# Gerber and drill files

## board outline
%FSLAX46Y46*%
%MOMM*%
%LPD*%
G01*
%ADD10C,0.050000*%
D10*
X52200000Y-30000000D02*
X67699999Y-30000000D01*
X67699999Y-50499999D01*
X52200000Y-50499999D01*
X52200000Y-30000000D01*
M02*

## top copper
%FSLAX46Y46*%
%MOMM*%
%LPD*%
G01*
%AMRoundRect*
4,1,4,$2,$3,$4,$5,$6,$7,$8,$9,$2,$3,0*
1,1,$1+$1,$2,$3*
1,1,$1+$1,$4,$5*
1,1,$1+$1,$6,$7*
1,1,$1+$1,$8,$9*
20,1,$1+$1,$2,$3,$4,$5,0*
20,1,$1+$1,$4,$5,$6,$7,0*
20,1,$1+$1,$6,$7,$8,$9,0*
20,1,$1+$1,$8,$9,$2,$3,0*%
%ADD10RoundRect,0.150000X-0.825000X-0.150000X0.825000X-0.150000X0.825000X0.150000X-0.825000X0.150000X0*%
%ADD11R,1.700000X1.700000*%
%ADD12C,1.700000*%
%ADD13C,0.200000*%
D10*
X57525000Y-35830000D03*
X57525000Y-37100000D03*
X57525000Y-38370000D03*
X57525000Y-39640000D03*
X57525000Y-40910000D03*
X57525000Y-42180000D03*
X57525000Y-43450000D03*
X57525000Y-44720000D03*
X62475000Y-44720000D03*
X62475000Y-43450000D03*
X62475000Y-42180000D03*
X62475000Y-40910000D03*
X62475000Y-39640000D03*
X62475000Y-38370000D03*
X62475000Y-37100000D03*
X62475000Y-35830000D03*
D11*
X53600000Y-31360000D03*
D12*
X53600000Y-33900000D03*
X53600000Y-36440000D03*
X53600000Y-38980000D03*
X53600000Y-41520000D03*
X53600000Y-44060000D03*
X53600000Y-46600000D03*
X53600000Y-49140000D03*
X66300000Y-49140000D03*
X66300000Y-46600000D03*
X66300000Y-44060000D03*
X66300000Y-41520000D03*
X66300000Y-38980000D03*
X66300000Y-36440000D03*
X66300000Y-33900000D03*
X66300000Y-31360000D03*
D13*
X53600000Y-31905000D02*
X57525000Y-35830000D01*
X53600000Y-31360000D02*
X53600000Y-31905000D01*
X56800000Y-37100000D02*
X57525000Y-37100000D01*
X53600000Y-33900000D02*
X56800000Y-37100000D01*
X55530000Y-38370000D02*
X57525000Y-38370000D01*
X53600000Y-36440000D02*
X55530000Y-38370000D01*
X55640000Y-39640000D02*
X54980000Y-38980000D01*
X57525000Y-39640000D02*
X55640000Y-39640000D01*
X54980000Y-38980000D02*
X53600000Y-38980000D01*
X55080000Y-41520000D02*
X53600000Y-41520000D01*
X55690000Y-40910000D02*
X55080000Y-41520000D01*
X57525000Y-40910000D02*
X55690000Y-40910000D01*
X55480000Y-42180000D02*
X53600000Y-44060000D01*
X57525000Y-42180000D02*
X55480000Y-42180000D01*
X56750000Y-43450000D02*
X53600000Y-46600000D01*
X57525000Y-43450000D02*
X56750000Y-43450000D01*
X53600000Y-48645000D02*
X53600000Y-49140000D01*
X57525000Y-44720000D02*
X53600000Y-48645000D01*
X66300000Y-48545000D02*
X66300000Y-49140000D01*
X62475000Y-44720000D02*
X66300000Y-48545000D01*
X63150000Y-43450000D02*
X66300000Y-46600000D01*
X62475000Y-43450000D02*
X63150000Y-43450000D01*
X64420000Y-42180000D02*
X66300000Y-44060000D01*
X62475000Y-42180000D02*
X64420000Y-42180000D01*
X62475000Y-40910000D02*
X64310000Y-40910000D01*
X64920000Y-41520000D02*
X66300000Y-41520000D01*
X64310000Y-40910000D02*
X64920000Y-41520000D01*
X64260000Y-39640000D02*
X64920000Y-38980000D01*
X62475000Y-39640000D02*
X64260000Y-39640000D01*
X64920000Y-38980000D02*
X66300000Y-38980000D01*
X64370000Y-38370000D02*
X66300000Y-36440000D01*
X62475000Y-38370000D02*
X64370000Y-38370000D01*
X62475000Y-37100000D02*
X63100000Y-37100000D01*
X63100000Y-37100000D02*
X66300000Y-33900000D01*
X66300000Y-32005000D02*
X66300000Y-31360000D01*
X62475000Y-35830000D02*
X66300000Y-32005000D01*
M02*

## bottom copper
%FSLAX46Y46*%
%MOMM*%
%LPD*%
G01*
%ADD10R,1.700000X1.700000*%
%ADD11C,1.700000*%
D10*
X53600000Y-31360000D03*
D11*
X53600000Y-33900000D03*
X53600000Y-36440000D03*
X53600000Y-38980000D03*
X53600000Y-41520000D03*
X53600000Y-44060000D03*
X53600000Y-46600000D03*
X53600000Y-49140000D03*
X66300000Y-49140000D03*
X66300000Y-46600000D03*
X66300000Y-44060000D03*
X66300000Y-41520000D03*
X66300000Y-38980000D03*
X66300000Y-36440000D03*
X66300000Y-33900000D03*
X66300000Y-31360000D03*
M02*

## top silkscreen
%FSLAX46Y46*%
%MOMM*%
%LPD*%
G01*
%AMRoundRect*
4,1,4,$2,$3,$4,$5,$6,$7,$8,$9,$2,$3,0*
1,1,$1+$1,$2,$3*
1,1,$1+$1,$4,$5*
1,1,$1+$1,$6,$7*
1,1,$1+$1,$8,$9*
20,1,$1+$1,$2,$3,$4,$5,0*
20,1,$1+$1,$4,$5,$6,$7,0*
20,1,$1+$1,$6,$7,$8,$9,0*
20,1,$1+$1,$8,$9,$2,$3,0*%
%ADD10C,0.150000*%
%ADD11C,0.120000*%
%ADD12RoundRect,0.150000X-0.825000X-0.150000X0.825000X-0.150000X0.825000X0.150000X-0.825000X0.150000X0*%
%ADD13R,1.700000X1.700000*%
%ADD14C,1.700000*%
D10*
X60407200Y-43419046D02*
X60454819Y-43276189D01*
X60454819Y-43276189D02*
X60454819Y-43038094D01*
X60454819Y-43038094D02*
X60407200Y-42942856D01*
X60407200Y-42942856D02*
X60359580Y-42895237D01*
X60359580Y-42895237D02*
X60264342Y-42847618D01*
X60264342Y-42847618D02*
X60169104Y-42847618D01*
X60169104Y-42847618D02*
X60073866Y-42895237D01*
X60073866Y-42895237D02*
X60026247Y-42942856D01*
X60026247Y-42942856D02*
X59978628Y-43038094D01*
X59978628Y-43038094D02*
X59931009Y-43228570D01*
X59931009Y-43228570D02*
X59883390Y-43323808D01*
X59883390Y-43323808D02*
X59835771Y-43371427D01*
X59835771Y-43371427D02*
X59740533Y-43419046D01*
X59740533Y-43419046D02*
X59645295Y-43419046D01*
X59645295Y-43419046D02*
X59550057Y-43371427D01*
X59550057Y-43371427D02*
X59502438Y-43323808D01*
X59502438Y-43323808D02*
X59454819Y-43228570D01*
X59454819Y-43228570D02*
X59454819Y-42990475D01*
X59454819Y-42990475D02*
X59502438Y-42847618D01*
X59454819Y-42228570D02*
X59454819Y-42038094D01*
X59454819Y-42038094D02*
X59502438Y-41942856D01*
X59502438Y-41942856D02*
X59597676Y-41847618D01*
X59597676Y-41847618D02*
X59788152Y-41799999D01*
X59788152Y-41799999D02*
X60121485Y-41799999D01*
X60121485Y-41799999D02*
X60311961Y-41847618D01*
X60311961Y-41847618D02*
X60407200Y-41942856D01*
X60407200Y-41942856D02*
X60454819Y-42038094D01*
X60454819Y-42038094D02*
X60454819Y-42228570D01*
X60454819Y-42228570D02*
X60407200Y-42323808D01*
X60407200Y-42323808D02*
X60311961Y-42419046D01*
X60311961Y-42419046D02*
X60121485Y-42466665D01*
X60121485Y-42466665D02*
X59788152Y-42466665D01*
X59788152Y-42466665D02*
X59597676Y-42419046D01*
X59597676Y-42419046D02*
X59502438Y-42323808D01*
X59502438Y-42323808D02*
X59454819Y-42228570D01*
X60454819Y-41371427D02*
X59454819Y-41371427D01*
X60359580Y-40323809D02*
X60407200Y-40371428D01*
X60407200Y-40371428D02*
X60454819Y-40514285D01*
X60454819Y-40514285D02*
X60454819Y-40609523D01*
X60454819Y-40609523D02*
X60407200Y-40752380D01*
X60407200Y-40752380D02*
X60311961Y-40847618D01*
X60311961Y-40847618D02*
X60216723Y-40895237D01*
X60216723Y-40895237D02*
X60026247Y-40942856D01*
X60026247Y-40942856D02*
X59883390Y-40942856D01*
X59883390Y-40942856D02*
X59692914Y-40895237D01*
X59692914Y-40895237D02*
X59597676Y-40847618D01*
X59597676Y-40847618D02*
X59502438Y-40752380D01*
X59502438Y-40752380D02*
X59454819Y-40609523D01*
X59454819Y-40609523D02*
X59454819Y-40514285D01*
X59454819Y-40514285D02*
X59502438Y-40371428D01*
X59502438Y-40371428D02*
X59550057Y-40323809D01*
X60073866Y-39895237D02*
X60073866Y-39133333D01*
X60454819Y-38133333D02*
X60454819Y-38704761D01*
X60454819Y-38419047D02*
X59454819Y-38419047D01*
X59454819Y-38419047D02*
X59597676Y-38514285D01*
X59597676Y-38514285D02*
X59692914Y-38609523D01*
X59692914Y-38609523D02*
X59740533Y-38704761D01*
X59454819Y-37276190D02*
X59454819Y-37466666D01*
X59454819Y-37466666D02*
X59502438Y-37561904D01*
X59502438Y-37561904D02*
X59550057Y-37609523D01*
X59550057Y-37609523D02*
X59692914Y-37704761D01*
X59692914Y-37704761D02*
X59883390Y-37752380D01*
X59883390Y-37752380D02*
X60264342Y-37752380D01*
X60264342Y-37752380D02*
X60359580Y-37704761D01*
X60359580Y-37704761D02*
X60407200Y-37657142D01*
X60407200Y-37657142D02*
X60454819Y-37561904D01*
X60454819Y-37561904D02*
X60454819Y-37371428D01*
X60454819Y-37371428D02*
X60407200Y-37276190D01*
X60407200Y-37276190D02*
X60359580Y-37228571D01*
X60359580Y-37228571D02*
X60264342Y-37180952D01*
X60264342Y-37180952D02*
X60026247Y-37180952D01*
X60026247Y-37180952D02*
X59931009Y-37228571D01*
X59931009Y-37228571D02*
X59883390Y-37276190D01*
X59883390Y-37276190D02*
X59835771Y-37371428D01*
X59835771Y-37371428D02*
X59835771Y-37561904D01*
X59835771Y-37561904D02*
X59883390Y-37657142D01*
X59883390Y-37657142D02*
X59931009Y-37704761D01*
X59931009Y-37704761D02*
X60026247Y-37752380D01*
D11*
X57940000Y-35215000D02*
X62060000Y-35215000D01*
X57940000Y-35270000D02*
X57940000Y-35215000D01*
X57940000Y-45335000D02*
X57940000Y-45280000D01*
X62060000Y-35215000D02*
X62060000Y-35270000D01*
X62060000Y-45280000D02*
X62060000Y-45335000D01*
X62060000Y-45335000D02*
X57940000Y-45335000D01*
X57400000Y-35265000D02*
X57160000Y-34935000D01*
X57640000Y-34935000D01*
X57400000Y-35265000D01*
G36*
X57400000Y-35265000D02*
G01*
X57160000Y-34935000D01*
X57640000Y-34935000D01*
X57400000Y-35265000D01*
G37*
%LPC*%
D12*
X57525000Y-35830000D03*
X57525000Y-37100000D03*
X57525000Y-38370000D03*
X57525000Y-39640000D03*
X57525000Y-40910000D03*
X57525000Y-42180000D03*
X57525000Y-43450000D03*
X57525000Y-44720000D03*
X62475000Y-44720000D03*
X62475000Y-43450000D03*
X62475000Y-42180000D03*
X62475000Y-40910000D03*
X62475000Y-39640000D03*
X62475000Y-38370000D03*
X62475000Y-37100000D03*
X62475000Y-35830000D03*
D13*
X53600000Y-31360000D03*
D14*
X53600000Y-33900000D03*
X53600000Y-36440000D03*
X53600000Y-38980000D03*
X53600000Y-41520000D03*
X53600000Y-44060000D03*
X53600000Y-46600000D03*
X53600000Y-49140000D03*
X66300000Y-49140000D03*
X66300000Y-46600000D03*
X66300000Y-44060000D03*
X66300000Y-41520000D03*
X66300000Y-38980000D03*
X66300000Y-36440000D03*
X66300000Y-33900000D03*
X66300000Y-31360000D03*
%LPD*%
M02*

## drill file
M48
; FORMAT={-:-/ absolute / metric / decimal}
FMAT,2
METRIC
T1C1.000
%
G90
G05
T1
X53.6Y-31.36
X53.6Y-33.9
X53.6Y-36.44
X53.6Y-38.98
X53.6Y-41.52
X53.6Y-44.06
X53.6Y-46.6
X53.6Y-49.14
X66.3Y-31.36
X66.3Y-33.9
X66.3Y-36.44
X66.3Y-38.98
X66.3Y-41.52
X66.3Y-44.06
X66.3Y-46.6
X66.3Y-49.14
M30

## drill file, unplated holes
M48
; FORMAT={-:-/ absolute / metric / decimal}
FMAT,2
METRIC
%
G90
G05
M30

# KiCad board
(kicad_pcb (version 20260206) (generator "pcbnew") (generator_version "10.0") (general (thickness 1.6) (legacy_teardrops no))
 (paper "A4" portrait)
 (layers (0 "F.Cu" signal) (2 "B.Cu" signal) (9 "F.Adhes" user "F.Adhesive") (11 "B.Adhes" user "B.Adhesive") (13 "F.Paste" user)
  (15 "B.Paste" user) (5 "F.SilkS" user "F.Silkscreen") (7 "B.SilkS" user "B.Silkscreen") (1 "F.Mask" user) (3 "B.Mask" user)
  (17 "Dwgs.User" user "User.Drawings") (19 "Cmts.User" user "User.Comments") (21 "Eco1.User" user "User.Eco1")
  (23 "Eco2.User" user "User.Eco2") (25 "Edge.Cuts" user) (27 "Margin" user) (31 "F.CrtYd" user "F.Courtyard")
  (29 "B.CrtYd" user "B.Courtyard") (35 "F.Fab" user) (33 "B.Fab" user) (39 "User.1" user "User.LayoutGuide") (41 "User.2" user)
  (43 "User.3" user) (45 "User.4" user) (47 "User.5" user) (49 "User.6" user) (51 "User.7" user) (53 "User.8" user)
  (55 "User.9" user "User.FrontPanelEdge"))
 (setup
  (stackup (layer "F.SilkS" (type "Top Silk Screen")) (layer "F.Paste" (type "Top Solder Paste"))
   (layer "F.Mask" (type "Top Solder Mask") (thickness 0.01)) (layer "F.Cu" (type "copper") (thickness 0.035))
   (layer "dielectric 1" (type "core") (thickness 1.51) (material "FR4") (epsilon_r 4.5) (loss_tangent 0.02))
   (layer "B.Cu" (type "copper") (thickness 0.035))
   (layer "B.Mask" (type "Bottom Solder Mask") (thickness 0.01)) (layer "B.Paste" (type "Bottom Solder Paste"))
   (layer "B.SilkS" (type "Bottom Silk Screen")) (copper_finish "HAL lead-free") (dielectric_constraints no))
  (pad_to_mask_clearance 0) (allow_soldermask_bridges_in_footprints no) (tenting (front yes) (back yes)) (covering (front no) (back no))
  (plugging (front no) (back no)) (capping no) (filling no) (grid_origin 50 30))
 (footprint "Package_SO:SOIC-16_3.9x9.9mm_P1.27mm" (layer "F.Cu") (at 60 40.275)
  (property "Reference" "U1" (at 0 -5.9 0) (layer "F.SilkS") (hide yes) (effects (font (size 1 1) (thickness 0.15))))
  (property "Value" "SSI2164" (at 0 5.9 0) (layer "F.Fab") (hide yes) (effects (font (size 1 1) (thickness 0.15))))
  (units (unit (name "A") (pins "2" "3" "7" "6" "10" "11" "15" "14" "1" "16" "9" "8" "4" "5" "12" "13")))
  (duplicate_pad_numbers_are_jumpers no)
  (fp_line (start -2.06 -5.06) (end 2.06 -5.06) (stroke (width 0.12) (type solid)) (layer "F.SilkS"))
  (fp_line (start -2.06 -5.005) (end -2.06 -5.06) (stroke (width 0.12) (type solid)) (layer "F.SilkS"))
  (fp_line (start -2.06 5.06) (end -2.06 5.005) (stroke (width 0.12) (type solid)) (layer "F.SilkS"))
  (fp_line (start 2.06 -5.06) (end 2.06 -5.005) (stroke (width 0.12) (type solid)) (layer "F.SilkS"))
  (fp_line (start 2.06 5.005) (end 2.06 5.06) (stroke (width 0.12) (type solid)) (layer "F.SilkS"))
  (fp_line (start 2.06 5.06) (end -2.06 5.06) (stroke (width 0.12) (type solid)) (layer "F.SilkS"))
  (fp_poly (pts (xy -2.6 -5.01) (xy -2.84 -5.34) (xy -2.36 -5.34)) (stroke (width 0.12) (type solid)) (fill yes) (layer "F.SilkS"))
  (pad "1" smd roundrect (at -2.475 -4.445) (size 1.95 0.6) (layers "F.Cu" "F.Mask" "F.Paste") (roundrect_rratio 0.25)
   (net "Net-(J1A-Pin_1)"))
  (pad "2" smd roundrect (at -2.475 -3.175) (size 1.95 0.6) (layers "F.Cu" "F.Mask" "F.Paste") (roundrect_rratio 0.25)
   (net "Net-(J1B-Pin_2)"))
  (pad "3" smd roundrect (at -2.475 -1.905) (size 1.95 0.6) (layers "F.Cu" "F.Mask" "F.Paste") (roundrect_rratio 0.25)
   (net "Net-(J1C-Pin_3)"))
  (pad "4" smd roundrect (at -2.475 -0.635) (size 1.95 0.6) (layers "F.Cu" "F.Mask" "F.Paste") (roundrect_rratio 0.25)
   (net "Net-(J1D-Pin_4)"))
  (pad "5" smd roundrect (at -2.475 0.635) (size 1.95 0.6) (layers "F.Cu" "F.Mask" "F.Paste") (roundrect_rratio 0.25)
   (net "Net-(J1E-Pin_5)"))
  (pad "6" smd roundrect (at -2.475 1.905) (size 1.95 0.6) (layers "F.Cu" "F.Mask" "F.Paste") (roundrect_rratio 0.25)
   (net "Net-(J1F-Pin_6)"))
  (pad "7" smd roundrect (at -2.475 3.175) (size 1.95 0.6) (layers "F.Cu" "F.Mask" "F.Paste") (roundrect_rratio 0.25)
   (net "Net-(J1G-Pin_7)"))
  (pad "8" smd roundrect (at -2.475 4.445) (size 1.95 0.6) (layers "F.Cu" "F.Mask" "F.Paste") (roundrect_rratio 0.25)
   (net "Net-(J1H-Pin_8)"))
  (pad "9" smd roundrect (at 2.475 4.445) (size 1.95 0.6) (layers "F.Cu" "F.Mask" "F.Paste") (roundrect_rratio 0.25) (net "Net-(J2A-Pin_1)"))
  (pad "10" smd roundrect (at 2.475 3.175) (size 1.95 0.6) (layers "F.Cu" "F.Mask" "F.Paste") (roundrect_rratio 0.25)
   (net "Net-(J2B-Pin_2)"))
  (pad "11" smd roundrect (at 2.475 1.905) (size 1.95 0.6) (layers "F.Cu" "F.Mask" "F.Paste") (roundrect_rratio 0.25)
   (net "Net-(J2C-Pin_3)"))
  (pad "12" smd roundrect (at 2.475 0.635) (size 1.95 0.6) (layers "F.Cu" "F.Mask" "F.Paste") (roundrect_rratio 0.25)
   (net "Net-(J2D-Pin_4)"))
  (pad "13" smd roundrect (at 2.475 -0.635) (size 1.95 0.6) (layers "F.Cu" "F.Mask" "F.Paste") (roundrect_rratio 0.25)
   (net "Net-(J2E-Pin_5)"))
  (pad "14" smd roundrect (at 2.475 -1.905) (size 1.95 0.6) (layers "F.Cu" "F.Mask" "F.Paste") (roundrect_rratio 0.25)
   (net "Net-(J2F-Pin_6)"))
  (pad "15" smd roundrect (at 2.475 -3.175) (size 1.95 0.6) (layers "F.Cu" "F.Mask" "F.Paste") (roundrect_rratio 0.25)
   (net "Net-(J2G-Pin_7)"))
  (pad "16" smd roundrect (at 2.475 -4.445) (size 1.95 0.6) (layers "F.Cu" "F.Mask" "F.Paste") (roundrect_rratio 0.25)
   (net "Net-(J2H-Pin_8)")))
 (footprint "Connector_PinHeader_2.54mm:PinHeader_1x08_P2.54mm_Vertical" (layer "B.Cu") (at 53.6 31.36 180)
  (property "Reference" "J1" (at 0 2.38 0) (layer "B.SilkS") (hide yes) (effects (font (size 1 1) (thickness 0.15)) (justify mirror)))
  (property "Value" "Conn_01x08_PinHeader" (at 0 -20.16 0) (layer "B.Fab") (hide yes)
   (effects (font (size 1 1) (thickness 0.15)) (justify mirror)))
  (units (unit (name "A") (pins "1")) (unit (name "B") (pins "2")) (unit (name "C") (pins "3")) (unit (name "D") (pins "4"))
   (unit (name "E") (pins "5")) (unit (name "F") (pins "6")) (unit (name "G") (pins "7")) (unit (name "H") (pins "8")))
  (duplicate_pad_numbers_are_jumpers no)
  (pad "1" thru_hole rect (at 0 0 180) (size 1.7 1.7) (drill 1) (layers "*.Cu" "*.Mask") (remove_unused_layers no) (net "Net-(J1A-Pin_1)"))
  (pad "2" thru_hole circle (at 0 -2.54 180) (size 1.7 1.7) (drill 1) (layers "*.Cu" "*.Mask") (remove_unused_layers no)
   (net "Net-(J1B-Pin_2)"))
  (pad "3" thru_hole circle (at 0 -5.08 180) (size 1.7 1.7) (drill 1) (layers "*.Cu" "*.Mask") (remove_unused_layers no)
   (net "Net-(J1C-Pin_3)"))
  (pad "4" thru_hole circle (at 0 -7.62 180) (size 1.7 1.7) (drill 1) (layers "*.Cu" "*.Mask") (remove_unused_layers no)
   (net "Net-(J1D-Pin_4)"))
  (pad "5" thru_hole circle (at 0 -10.16 180) (size 1.7 1.7) (drill 1) (layers "*.Cu" "*.Mask") (remove_unused_layers no)
   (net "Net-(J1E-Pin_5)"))
  (pad "6" thru_hole circle (at 0 -12.7 180) (size 1.7 1.7) (drill 1) (layers "*.Cu" "*.Mask") (remove_unused_layers no)
   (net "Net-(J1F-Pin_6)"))
  (pad "7" thru_hole circle (at 0 -15.24 180) (size 1.7 1.7) (drill 1) (layers "*.Cu" "*.Mask") (remove_unused_layers no)
   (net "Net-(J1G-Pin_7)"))
  (pad "8" thru_hole circle (at 0 -17.78 180) (size 1.7 1.7) (drill 1) (layers "*.Cu" "*.Mask") (remove_unused_layers no)
   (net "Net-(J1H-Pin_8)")))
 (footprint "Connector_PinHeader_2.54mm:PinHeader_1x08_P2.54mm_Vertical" (layer "B.Cu") (at 66.3 49.14)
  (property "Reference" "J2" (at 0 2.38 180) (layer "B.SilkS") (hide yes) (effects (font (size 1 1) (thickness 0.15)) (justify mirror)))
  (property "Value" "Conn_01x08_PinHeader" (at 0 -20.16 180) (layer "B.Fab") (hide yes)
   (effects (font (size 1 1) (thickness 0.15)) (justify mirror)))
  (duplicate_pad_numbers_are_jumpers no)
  (pad "1" thru_hole circle (at 0 0) (size 1.7 1.7) (drill 1) (layers "*.Cu" "*.Mask") (remove_unused_layers no) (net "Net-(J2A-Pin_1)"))
  (pad "2" thru_hole circle (at 0 -2.54) (size 1.7 1.7) (drill 1) (layers "*.Cu" "*.Mask") (remove_unused_layers no) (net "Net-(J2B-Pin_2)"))
  (pad "3" thru_hole circle (at 0 -5.08) (size 1.7 1.7) (drill 1) (layers "*.Cu" "*.Mask") (remove_unused_layers no) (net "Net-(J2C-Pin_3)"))
  (pad "4" thru_hole circle (at 0 -7.62) (size 1.7 1.7) (drill 1) (layers "*.Cu" "*.Mask") (remove_unused_layers no) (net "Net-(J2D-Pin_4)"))
  (pad "5" thru_hole circle (at 0 -10.16) (size 1.7 1.7) (drill 1) (layers "*.Cu" "*.Mask") (remove_unused_layers no)
   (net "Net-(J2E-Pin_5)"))
  (pad "6" thru_hole circle (at 0 -12.7) (size 1.7 1.7) (drill 1) (layers "*.Cu" "*.Mask") (remove_unused_layers no) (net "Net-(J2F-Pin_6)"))
  (pad "7" thru_hole circle (at 0 -15.24) (size 1.7 1.7) (drill 1) (layers "*.Cu" "*.Mask") (remove_unused_layers no)
   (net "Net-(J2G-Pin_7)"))
  (pad "8" thru_hole circle (at 0 -17.78) (size 1.7 1.7) (drill 1) (layers "*.Cu" "*.Mask") (remove_unused_layers no)
   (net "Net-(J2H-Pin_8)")))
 (gr_rect (start 52.2 30) (end 67.699999 50.499999) (stroke (width 0.05) (type default)) (fill no) (layer "Edge.Cuts"))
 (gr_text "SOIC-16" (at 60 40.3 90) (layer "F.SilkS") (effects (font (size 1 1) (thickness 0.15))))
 (segment (start 53.6 31.905) (end 57.525 35.83) (width 0.2) (layer "F.Cu") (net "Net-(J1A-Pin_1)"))
 (segment (start 53.6 31.36) (end 53.6 31.905) (width 0.2) (layer "F.Cu") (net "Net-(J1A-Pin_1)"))
 (segment (start 56.8 37.1) (end 57.525 37.1) (width 0.2) (layer "F.Cu") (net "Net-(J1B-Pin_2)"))
 (segment (start 53.6 33.9) (end 56.8 37.1) (width 0.2) (layer "F.Cu") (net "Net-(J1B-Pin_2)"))
 (segment (start 55.53 38.37) (end 57.525 38.37) (width 0.2) (layer "F.Cu") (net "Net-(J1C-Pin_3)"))
 (segment (start 53.6 36.44) (end 55.53 38.37) (width 0.2) (layer "F.Cu") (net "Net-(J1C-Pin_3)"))
 (segment (start 55.64 39.64) (end 54.98 38.98) (width 0.2) (layer "F.Cu") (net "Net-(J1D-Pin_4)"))
 (segment (start 57.525 39.64) (end 55.64 39.64) (width 0.2) (layer "F.Cu") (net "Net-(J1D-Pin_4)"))
 (segment (start 54.98 38.98) (end 53.6 38.98) (width 0.2) (layer "F.Cu") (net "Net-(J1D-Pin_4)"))
 (segment (start 55.08 41.52) (end 53.6 41.52) (width 0.2) (layer "F.Cu") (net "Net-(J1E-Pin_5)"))
 (segment (start 55.69 40.91) (end 55.08 41.52) (width 0.2) (layer "F.Cu") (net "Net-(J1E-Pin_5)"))
 (segment (start 57.525 40.91) (end 55.69 40.91) (width 0.2) (layer "F.Cu") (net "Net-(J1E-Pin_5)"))
 (segment (start 55.48 42.18) (end 53.6 44.06) (width 0.2) (layer "F.Cu") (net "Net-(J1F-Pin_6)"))
 (segment (start 57.525 42.18) (end 55.48 42.18) (width 0.2) (layer "F.Cu") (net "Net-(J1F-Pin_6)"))
 (segment (start 56.75 43.45) (end 53.6 46.6) (width 0.2) (layer "F.Cu") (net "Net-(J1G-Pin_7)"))
 (segment (start 57.525 43.45) (end 56.75 43.45) (width 0.2) (layer "F.Cu") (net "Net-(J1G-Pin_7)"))
 (segment (start 53.6 48.645) (end 53.6 49.14) (width 0.2) (layer "F.Cu") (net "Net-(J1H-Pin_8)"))
 (segment (start 57.525 44.72) (end 53.6 48.645) (width 0.2) (layer "F.Cu") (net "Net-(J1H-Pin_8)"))
 (segment (start 66.3 48.545) (end 66.3 49.14) (width 0.2) (layer "F.Cu") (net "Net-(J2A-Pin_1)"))
 (segment (start 62.475 44.72) (end 66.3 48.545) (width 0.2) (layer "F.Cu") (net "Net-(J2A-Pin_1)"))
 (segment (start 63.15 43.45) (end 66.3 46.6) (width 0.2) (layer "F.Cu") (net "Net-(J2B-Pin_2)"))
 (segment (start 62.475 43.45) (end 63.15 43.45) (width 0.2) (layer "F.Cu") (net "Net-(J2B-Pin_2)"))
 (segment (start 64.42 42.18) (end 66.3 44.06) (width 0.2) (layer "F.Cu") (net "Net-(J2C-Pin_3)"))
 (segment (start 62.475 42.18) (end 64.42 42.18) (width 0.2) (layer "F.Cu") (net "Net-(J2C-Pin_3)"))
 (segment (start 62.475 40.91) (end 64.31 40.91) (width 0.2) (layer "F.Cu") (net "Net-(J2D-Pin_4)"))
 (segment (start 64.92 41.52) (end 66.3 41.52) (width 0.2) (layer "F.Cu") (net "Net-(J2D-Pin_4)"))
 (segment (start 64.31 40.91) (end 64.92 41.52) (width 0.2) (layer "F.Cu") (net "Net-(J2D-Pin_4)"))
 (segment (start 64.26 39.64) (end 64.92 38.98) (width 0.2) (layer "F.Cu") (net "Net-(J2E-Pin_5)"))
 (segment (start 62.475 39.64) (end 64.26 39.64) (width 0.2) (layer "F.Cu") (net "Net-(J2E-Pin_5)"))
 (segment (start 64.92 38.98) (end 66.3 38.98) (width 0.2) (layer "F.Cu") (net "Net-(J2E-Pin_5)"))
 (segment (start 64.37 38.37) (end 66.3 36.44) (width 0.2) (layer "F.Cu") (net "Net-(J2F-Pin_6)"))
 (segment (start 62.475 38.37) (end 64.37 38.37) (width 0.2) (layer "F.Cu") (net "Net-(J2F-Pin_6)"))
 (segment (start 62.475 37.1) (end 63.1 37.1) (width 0.2) (layer "F.Cu") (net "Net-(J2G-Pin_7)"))
 (segment (start 63.1 37.1) (end 66.3 33.9) (width 0.2) (layer "F.Cu") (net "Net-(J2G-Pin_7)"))
 (segment (start 66.3 32.005) (end 66.3 31.36) (width 0.2) (layer "F.Cu") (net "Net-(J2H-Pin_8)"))
 (segment (start 62.475 35.83) (end 66.3 32.005) (width 0.2) (layer "F.Cu") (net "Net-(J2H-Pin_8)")))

